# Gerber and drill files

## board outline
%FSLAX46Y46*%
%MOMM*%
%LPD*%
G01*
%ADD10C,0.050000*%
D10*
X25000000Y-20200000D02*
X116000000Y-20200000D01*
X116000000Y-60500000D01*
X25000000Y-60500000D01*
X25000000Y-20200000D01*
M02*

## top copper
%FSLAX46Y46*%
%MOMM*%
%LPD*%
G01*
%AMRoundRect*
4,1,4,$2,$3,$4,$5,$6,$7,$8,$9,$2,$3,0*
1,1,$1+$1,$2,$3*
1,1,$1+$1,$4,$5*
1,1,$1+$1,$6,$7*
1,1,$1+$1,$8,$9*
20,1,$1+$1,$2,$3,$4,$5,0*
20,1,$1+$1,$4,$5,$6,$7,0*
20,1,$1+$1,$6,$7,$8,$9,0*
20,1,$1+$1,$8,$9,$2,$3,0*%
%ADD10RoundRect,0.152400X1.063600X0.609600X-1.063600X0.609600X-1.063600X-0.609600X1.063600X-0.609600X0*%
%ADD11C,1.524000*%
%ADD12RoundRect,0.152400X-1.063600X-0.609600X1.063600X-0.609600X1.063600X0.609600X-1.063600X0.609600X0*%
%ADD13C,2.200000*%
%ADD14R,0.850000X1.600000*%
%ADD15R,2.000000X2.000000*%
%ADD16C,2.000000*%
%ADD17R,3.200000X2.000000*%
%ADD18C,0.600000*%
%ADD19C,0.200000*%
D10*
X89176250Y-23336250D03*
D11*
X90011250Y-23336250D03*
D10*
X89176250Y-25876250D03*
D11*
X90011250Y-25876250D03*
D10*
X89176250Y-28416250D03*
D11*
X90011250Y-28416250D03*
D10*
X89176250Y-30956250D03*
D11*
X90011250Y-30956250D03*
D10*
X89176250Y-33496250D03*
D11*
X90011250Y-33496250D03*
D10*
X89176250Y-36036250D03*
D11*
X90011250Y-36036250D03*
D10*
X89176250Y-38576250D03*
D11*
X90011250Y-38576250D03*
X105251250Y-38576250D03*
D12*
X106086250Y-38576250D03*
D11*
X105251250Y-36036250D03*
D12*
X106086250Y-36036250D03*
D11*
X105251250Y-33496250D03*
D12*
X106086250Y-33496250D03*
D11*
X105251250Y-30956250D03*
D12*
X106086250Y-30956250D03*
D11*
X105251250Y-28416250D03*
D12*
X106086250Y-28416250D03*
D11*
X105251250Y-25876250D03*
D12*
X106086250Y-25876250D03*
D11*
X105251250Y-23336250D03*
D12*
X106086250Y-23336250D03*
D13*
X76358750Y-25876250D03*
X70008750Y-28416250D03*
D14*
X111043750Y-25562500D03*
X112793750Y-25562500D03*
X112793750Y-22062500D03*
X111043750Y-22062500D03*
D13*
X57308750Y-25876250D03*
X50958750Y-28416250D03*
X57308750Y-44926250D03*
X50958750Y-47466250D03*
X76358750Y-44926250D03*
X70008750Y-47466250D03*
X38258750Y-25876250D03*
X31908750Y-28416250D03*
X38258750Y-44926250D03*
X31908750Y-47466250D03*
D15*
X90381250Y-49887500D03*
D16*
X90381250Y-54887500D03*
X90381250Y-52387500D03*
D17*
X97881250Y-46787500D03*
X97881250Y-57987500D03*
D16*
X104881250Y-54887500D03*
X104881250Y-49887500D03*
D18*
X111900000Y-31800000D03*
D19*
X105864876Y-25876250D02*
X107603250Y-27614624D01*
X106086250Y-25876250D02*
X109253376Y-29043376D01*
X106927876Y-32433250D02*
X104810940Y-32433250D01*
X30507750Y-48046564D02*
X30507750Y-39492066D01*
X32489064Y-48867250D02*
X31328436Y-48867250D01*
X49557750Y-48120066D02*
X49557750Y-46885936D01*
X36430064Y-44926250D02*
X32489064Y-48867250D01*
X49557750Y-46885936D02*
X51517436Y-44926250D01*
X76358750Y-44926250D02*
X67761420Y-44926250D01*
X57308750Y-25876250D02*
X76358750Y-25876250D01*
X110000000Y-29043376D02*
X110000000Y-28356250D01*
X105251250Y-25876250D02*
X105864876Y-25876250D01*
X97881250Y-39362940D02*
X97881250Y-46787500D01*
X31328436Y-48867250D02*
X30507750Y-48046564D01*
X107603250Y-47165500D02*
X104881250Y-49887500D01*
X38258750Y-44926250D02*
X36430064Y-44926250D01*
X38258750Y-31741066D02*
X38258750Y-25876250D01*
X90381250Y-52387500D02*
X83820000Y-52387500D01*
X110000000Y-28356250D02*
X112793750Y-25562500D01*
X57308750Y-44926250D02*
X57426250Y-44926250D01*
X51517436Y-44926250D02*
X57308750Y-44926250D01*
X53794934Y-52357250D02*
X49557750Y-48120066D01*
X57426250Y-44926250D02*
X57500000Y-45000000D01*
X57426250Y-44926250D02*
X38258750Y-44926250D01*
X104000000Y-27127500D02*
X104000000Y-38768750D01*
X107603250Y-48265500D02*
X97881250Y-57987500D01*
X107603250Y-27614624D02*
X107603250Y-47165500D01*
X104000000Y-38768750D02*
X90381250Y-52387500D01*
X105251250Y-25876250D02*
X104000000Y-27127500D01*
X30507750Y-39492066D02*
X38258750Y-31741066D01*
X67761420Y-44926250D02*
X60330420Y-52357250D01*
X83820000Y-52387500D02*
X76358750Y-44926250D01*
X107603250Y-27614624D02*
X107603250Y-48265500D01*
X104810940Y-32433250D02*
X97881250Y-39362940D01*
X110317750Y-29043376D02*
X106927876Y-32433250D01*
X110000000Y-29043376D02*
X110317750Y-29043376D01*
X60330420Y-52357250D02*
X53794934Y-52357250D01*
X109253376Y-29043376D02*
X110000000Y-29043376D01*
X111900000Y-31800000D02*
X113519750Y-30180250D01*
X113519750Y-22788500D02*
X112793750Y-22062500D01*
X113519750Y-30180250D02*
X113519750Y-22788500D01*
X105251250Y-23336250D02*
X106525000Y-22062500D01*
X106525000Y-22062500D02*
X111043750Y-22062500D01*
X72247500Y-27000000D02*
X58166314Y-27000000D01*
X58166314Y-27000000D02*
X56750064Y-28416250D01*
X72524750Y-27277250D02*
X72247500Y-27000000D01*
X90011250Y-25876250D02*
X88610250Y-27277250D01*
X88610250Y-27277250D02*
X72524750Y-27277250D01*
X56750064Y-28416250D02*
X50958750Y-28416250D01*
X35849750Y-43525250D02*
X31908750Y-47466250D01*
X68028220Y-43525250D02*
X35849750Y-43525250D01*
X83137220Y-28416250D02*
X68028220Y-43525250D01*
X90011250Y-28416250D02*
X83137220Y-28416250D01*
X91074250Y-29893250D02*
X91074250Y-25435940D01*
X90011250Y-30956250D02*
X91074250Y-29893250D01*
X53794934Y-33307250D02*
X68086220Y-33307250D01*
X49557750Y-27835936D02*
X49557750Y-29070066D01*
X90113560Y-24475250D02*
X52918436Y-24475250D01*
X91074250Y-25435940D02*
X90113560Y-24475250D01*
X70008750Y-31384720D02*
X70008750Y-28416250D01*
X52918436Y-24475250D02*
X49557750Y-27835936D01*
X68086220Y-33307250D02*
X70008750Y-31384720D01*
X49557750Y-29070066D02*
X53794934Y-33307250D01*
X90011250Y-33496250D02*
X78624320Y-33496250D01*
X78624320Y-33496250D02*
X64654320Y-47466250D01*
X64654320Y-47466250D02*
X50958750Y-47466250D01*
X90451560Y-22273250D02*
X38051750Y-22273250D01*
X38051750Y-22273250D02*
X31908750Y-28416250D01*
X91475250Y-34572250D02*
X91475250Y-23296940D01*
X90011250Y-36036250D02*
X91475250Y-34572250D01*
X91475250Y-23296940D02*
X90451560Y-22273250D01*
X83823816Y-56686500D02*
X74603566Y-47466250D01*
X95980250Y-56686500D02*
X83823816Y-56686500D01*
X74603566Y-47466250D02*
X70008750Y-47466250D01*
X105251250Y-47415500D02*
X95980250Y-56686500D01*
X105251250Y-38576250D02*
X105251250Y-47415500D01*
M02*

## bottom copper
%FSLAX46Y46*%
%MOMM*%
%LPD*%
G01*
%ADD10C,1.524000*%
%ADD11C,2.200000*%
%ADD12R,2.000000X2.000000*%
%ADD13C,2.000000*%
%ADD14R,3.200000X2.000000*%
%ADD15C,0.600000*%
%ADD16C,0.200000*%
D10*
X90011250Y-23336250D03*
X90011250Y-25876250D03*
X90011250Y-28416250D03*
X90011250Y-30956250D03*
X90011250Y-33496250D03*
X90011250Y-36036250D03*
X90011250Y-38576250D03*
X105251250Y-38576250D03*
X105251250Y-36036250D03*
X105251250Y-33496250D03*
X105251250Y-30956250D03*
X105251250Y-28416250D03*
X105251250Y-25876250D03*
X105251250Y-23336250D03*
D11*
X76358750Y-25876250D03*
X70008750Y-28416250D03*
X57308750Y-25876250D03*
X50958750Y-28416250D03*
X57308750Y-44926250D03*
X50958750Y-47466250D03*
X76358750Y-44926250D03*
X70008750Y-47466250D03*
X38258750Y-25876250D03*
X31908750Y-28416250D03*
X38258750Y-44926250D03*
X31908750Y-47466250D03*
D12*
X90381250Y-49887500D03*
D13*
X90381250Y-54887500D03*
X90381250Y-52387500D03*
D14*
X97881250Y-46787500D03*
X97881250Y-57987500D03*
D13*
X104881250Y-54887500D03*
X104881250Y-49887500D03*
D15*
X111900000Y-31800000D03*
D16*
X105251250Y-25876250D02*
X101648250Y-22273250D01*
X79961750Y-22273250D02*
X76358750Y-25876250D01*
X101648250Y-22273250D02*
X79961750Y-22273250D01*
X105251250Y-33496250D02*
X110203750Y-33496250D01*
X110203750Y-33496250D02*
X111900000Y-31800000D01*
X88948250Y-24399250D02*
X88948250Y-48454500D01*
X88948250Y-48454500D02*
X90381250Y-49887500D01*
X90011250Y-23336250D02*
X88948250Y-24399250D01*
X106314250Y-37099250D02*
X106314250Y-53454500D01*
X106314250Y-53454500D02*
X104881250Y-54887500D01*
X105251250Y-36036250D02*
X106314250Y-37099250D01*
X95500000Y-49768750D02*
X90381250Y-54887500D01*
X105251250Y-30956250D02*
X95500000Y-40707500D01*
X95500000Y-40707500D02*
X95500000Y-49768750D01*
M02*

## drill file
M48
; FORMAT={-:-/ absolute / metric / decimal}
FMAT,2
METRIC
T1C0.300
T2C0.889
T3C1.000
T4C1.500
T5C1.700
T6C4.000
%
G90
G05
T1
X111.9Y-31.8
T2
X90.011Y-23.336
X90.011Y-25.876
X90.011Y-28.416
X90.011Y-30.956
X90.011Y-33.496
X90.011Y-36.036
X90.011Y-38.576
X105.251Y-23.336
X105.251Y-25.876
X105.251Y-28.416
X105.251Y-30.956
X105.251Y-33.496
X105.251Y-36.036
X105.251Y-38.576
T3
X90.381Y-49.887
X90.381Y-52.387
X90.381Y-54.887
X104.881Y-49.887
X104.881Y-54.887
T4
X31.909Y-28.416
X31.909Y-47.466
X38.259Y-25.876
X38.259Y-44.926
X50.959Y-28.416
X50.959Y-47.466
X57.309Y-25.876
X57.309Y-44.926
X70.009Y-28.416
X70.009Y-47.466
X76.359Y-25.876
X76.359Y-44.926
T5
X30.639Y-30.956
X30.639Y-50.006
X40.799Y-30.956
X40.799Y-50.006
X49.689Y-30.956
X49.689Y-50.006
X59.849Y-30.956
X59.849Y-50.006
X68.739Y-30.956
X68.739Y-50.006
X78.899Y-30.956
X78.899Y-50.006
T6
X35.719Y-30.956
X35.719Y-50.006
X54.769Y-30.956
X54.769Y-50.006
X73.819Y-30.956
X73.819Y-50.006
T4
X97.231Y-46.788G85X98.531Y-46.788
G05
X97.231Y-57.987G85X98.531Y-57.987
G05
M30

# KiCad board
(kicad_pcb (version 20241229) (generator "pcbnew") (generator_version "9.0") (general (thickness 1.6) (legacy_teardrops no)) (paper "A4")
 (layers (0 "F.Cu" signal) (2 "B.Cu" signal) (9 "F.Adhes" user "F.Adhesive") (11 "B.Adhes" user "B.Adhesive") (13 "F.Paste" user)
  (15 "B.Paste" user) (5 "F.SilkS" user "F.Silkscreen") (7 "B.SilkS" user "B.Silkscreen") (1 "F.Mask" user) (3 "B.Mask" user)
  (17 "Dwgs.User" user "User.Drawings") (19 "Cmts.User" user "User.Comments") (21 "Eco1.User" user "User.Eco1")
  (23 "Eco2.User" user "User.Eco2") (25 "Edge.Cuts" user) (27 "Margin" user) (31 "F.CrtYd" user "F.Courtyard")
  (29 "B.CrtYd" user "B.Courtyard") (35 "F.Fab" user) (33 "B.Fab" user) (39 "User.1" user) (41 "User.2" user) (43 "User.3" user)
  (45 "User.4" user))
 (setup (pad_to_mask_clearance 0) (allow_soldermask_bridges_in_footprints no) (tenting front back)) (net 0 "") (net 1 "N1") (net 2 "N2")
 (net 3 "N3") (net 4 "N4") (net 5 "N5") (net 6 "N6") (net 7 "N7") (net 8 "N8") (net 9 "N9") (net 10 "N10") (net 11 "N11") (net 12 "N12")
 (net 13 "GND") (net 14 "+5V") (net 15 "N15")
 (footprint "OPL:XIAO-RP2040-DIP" (layer "F.Cu") (at 97.63125 30.95625)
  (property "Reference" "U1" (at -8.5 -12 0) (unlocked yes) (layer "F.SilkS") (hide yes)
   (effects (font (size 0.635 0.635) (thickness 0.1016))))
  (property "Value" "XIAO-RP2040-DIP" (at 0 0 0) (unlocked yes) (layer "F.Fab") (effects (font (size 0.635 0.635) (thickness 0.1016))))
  (pad "1" smd roundrect (at -8.455 -7.62 180) (size 2.432 1.524) (layers "F.Cu" "F.Mask") (roundrect_rratio 0.1) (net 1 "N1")
   (thermal_bridge_angle 45))
  (pad "1" thru_hole circle (at -7.62 -7.62 180) (size 1.524 1.524) (drill 0.889) (layers "*.Cu" "*.Mask") (remove_unused_layers no)
   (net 1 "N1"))
  (pad "2" smd roundrect (at -8.455 -5.08 180) (size 2.432 1.524) (layers "F.Cu" "F.Mask") (roundrect_rratio 0.1) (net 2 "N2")
   (thermal_bridge_angle 45))
  (pad "2" thru_hole circle (at -7.62 -5.08 180) (size 1.524 1.524) (drill 0.889) (layers "*.Cu" "*.Mask") (remove_unused_layers no)
   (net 2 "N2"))
  (pad "3" smd roundrect (at -8.455 -2.54 180) (size 2.432 1.524) (layers "F.Cu" "F.Mask") (roundrect_rratio 0.1) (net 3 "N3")
   (thermal_bridge_angle 45))
  (pad "3" thru_hole circle (at -7.62 -2.54 180) (size 1.524 1.524) (drill 0.889) (layers "*.Cu" "*.Mask") (remove_unused_layers no)
   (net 3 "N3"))
  (pad "4" smd roundrect (at -8.455 0 180) (size 2.432 1.524) (layers "F.Cu" "F.Mask") (roundrect_rratio 0.1) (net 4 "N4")
   (thermal_bridge_angle 45))
  (pad "4" thru_hole circle (at -7.62 0 180) (size 1.524 1.524) (drill 0.889) (layers "*.Cu" "*.Mask") (remove_unused_layers no)
   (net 4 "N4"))
  (pad "5" smd roundrect (at -8.455 2.54 180) (size 2.432 1.524) (layers "F.Cu" "F.Mask") (roundrect_rratio 0.1) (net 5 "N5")
   (thermal_bridge_angle 45))
  (pad "5" thru_hole circle (at -7.62 2.54 180) (size 1.524 1.524) (drill 0.889) (layers "*.Cu" "*.Mask") (remove_unused_layers no)
   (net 5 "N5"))
  (pad "6" smd roundrect (at -8.455 5.08 180) (size 2.432 1.524) (layers "F.Cu" "F.Mask") (roundrect_rratio 0.1) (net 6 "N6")
   (thermal_bridge_angle 45))
  (pad "6" thru_hole circle (at -7.62 5.08 180) (size 1.524 1.524) (drill 0.889) (layers "*.Cu" "*.Mask") (remove_unused_layers no)
   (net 6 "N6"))
  (pad "7" smd roundrect (at -8.455 7.62 180) (size 2.432 1.524) (layers "F.Cu" "F.Mask") (roundrect_rratio 0.1) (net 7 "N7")
   (thermal_bridge_angle 45))
  (pad "7" thru_hole circle (at -7.62 7.62 180) (size 1.524 1.524) (drill 0.889) (layers "*.Cu" "*.Mask") (remove_unused_layers no)
   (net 7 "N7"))
  (pad "8" thru_hole circle (at 7.62 7.62) (size 1.524 1.524) (drill 0.889) (layers "*.Cu" "*.Mask") (remove_unused_layers no) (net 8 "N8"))
  (pad "8" smd roundrect (at 8.455 7.62) (size 2.432 1.524) (layers "F.Cu" "F.Mask") (roundrect_rratio 0.1) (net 8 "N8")
   (thermal_bridge_angle 45))
  (pad "9" thru_hole circle (at 7.62 5.08) (size 1.524 1.524) (drill 0.889) (layers "*.Cu" "*.Mask") (remove_unused_layers no) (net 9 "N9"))
  (pad "9" smd roundrect (at 8.455 5.08) (size 2.432 1.524) (layers "F.Cu" "F.Mask") (roundrect_rratio 0.1) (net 9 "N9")
   (thermal_bridge_angle 45))
  (pad "10" thru_hole circle (at 7.62 2.54) (size 1.524 1.524) (drill 0.889) (layers "*.Cu" "*.Mask") (remove_unused_layers no)
   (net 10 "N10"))
  (pad "10" smd roundrect (at 8.455 2.54) (size 2.432 1.524) (layers "F.Cu" "F.Mask") (roundrect_rratio 0.1) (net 10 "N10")
   (thermal_bridge_angle 45))
  (pad "11" thru_hole circle (at 7.62 0) (size 1.524 1.524) (drill 0.889) (layers "*.Cu" "*.Mask") (remove_unused_layers no) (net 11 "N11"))
  (pad "11" smd roundrect (at 8.455 0) (size 2.432 1.524) (layers "F.Cu" "F.Mask") (roundrect_rratio 0.1) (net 11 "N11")
   (thermal_bridge_angle 45))
  (pad "12" thru_hole circle (at 7.62 -2.54) (size 1.524 1.524) (drill 0.889) (layers "*.Cu" "*.Mask") (remove_unused_layers no)
   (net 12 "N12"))
  (pad "12" smd roundrect (at 8.455 -2.54) (size 2.432 1.524) (layers "F.Cu" "F.Mask") (roundrect_rratio 0.1) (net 12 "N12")
   (thermal_bridge_angle 45))
  (pad "13" thru_hole circle (at 7.62 -5.08) (size 1.524 1.524) (drill 0.889) (layers "*.Cu" "*.Mask") (remove_unused_layers no)
   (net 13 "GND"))
  (pad "13" smd roundrect (at 8.455 -5.08) (size 2.432 1.524) (layers "F.Cu" "F.Mask") (roundrect_rratio 0.1) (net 13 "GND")
   (thermal_bridge_angle 45))
  (pad "14" thru_hole circle (at 7.62 -7.62) (size 1.524 1.524) (drill 0.889) (layers "*.Cu" "*.Mask") (remove_unused_layers no)
   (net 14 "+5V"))
  (pad "14" smd roundrect (at 8.455 -7.62) (size 2.432 1.524) (layers "F.Cu" "F.Mask") (roundrect_rratio 0.1) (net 14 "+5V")
   (thermal_bridge_angle 45)))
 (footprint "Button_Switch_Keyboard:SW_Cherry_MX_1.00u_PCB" (layer "F.Cu") (at 76.35875 25.87625)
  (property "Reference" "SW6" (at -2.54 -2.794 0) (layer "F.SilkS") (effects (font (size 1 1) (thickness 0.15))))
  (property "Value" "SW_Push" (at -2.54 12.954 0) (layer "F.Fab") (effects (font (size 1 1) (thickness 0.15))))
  (pad "" np_thru_hole circle (at -7.62 5.08) (size 1.7 1.7) (drill 1.7) (layers "*.Cu" "*.Mask"))
  (pad "" np_thru_hole circle (at -2.54 5.08) (size 4 4) (drill 4) (layers "*.Cu" "*.Mask"))
  (pad "" np_thru_hole circle (at 2.54 5.08) (size 1.7 1.7) (drill 1.7) (layers "*.Cu" "*.Mask"))
  (pad "1" thru_hole circle (at 0 0) (size 2.2 2.2) (drill 1.5) (layers "*.Cu" "*.Mask") (remove_unused_layers no) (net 13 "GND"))
  (pad "2" thru_hole circle (at -6.35 2.54) (size 2.2 2.2) (drill 1.5) (layers "*.Cu" "*.Mask") (remove_unused_layers no) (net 4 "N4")))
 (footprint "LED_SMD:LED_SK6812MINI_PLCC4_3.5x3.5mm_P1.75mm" (layer "F.Cu") (at 111.91875 23.8125 90)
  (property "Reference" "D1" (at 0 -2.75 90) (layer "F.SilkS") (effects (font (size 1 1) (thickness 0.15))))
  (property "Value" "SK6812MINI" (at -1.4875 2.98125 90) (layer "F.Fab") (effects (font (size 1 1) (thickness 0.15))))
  (pad "1" smd rect (at -1.75 -0.875 90) (size 1.6 0.85) (layers "F.Cu" "F.Mask" "F.Paste") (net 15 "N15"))
  (pad "2" smd rect (at -1.75 0.875 90) (size 1.6 0.85) (layers "F.Cu" "F.Mask" "F.Paste") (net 13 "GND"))
  (pad "3" smd rect (at 1.75 0.875 90) (size 1.6 0.85) (layers "F.Cu" "F.Mask" "F.Paste") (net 10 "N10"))
  (pad "4" smd rect (at 1.75 -0.875 90) (size 1.6 0.85) (layers "F.Cu" "F.Mask" "F.Paste") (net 14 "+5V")))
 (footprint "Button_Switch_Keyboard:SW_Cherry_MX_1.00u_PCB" (layer "F.Cu") (at 57.30875 25.87625)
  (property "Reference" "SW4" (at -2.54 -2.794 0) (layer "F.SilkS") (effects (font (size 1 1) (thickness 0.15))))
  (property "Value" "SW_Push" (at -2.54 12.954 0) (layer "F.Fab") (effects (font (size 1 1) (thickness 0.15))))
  (pad "" np_thru_hole circle (at -7.62 5.08) (size 1.7 1.7) (drill 1.7) (layers "*.Cu" "*.Mask"))
  (pad "" np_thru_hole circle (at -2.54 5.08) (size 4 4) (drill 4) (layers "*.Cu" "*.Mask"))
  (pad "" np_thru_hole circle (at 2.54 5.08) (size 1.7 1.7) (drill 1.7) (layers "*.Cu" "*.Mask"))
  (pad "1" thru_hole circle (at 0 0) (size 2.2 2.2) (drill 1.5) (layers "*.Cu" "*.Mask") (remove_unused_layers no) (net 13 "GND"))
  (pad "2" thru_hole circle (at -6.35 2.54) (size 2.2 2.2) (drill 1.5) (layers "*.Cu" "*.Mask") (remove_unused_layers no) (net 2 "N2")))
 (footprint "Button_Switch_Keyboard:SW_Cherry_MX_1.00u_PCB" (layer "F.Cu") (at 57.30875 44.92625)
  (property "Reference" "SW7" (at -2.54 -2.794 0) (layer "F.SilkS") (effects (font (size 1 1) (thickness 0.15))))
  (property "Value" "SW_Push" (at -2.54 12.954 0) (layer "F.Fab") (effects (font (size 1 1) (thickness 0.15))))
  (pad "" np_thru_hole circle (at -7.62 5.08) (size 1.7 1.7) (drill 1.7) (layers "*.Cu" "*.Mask"))
  (pad "" np_thru_hole circle (at -2.54 5.08) (size 4 4) (drill 4) (layers "*.Cu" "*.Mask"))
  (pad "" np_thru_hole circle (at 2.54 5.08) (size 1.7 1.7) (drill 1.7) (layers "*.Cu" "*.Mask"))
  (pad "1" thru_hole circle (at 0 0) (size 2.2 2.2) (drill 1.5) (layers "*.Cu" "*.Mask") (remove_unused_layers no) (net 13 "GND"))
  (pad "2" thru_hole circle (at -6.35 2.54) (size 2.2 2.2) (drill 1.5) (layers "*.Cu" "*.Mask") (remove_unused_layers no) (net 5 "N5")))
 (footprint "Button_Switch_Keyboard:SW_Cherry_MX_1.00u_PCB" (layer "F.Cu") (at 76.35875 44.92625)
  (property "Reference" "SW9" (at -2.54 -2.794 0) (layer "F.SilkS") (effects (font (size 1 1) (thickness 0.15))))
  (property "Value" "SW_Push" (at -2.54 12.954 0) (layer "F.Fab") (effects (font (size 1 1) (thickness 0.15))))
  (pad "" np_thru_hole circle (at -7.62 5.08) (size 1.7 1.7) (drill 1.7) (layers "*.Cu" "*.Mask"))
  (pad "" np_thru_hole circle (at -2.54 5.08) (size 4 4) (drill 4) (layers "*.Cu" "*.Mask"))
  (pad "" np_thru_hole circle (at 2.54 5.08) (size 1.7 1.7) (drill 1.7) (layers "*.Cu" "*.Mask"))
  (pad "1" thru_hole circle (at 0 0) (size 2.2 2.2) (drill 1.5) (layers "*.Cu" "*.Mask") (remove_unused_layers no) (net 13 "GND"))
  (pad "2" thru_hole circle (at -6.35 2.54) (size 2.2 2.2) (drill 1.5) (layers "*.Cu" "*.Mask") (remove_unused_layers no) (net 8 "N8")))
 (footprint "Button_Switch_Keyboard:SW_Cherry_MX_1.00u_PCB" (layer "F.Cu") (at 38.25875 25.87625)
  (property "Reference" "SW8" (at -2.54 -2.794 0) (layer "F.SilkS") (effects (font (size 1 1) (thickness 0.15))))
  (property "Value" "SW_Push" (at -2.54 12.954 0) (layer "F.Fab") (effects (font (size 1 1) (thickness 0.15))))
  (pad "" np_thru_hole circle (at -7.62 5.08) (size 1.7 1.7) (drill 1.7) (layers "*.Cu" "*.Mask"))
  (pad "" np_thru_hole circle (at -2.54 5.08) (size 4 4) (drill 4) (layers "*.Cu" "*.Mask"))
  (pad "" np_thru_hole circle (at 2.54 5.08) (size 1.7 1.7) (drill 1.7) (layers "*.Cu" "*.Mask"))
  (pad "1" thru_hole circle (at 0 0) (size 2.2 2.2) (drill 1.5) (layers "*.Cu" "*.Mask") (remove_unused_layers no) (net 13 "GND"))
  (pad "2" thru_hole circle (at -6.35 2.54) (size 2.2 2.2) (drill 1.5) (layers "*.Cu" "*.Mask") (remove_unused_layers no) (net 6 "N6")))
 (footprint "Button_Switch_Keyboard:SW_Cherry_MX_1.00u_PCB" (layer "F.Cu") (at 38.25875 44.92625)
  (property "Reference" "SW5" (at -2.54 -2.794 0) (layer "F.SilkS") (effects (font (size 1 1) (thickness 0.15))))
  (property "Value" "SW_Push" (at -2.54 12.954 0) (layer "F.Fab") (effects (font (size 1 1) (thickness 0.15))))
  (pad "" np_thru_hole circle (at -7.62 5.08) (size 1.7 1.7) (drill 1.7) (layers "*.Cu" "*.Mask"))
  (pad "" np_thru_hole circle (at -2.54 5.08) (size 4 4) (drill 4) (layers "*.Cu" "*.Mask"))
  (pad "" np_thru_hole circle (at 2.54 5.08) (size 1.7 1.7) (drill 1.7) (layers "*.Cu" "*.Mask"))
  (pad "1" thru_hole circle (at 0 0) (size 2.2 2.2) (drill 1.5) (layers "*.Cu" "*.Mask") (remove_unused_layers no) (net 13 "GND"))
  (pad "2" thru_hole circle (at -6.35 2.54) (size 2.2 2.2) (drill 1.5) (layers "*.Cu" "*.Mask") (remove_unused_layers no) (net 3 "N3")))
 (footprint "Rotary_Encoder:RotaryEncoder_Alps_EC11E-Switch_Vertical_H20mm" (layer "F.Cu") (at 90.38125 49.8875)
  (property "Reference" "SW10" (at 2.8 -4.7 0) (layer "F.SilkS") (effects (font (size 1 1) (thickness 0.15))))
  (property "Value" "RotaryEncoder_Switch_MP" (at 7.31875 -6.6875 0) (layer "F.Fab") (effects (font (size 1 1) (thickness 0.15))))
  (pad "A" thru_hole rect (at 0 0) (size 2 2) (drill 1) (layers "*.Cu" "*.Mask") (remove_unused_layers no) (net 1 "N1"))
  (pad "B" thru_hole circle (at 0 5) (size 2 2) (drill 1) (layers "*.Cu" "*.Mask") (remove_unused_layers no) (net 11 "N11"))
  (pad "C" thru_hole circle (at 0 2.5) (size 2 2) (drill 1) (layers "*.Cu" "*.Mask") (remove_unused_layers no) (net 13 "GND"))
  (pad "MP" thru_hole rect (at 7.5 -3.1) (size 3.2 2) (drill oval 2.8 1.5) (layers "*.Cu" "*.Mask") (remove_unused_layers no) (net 13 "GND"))
  (pad "MP" thru_hole rect (at 7.5 8.1) (size 3.2 2) (drill oval 2.8 1.5) (layers "*.Cu" "*.Mask") (remove_unused_layers no) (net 13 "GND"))
  (pad "S1" thru_hole circle (at 14.5 5) (size 2 2) (drill 1) (layers "*.Cu" "*.Mask") (remove_unused_layers no) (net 9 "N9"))
  (pad "S2" thru_hole circle (at 14.5 0) (size 2 2) (drill 1) (layers "*.Cu" "*.Mask") (remove_unused_layers no) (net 13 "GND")))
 (gr_rect (start 25 20.2) (end 116 60.5) (stroke (width 0.05) (type default)) (fill no) (layer "Edge.Cuts"))
 (segment (start 105.864876 25.87625) (end 107.60325 27.614624) (width 0.2) (layer "F.Cu") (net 13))
 (segment (start 106.08625 25.87625) (end 109.253376 29.043376) (width 0.2) (layer "F.Cu") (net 13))
 (segment (start 106.927876 32.43325) (end 104.81094 32.43325) (width 0.2) (layer "F.Cu") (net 13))
 (segment (start 30.50775 48.046564) (end 30.50775 39.492066) (width 0.2) (layer "F.Cu") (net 13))
 (segment (start 32.489064 48.86725) (end 31.328436 48.86725) (width 0.2) (layer "F.Cu") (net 13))
 (segment (start 49.55775 48.120066) (end 49.55775 46.885936) (width 0.2) (layer "F.Cu") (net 13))
 (segment (start 36.430064 44.92625) (end 32.489064 48.86725) (width 0.2) (layer "F.Cu") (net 13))
 (segment (start 49.55775 46.885936) (end 51.517436 44.92625) (width 0.2) (layer "F.Cu") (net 13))
 (segment (start 76.35875 44.92625) (end 67.76142 44.92625) (width 0.2) (layer "F.Cu") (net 13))
 (segment (start 57.30875 25.87625) (end 76.35875 25.87625) (width 0.2) (layer "F.Cu") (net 13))
 (segment (start 110 29.043376) (end 110 28.35625) (width 0.2) (layer "F.Cu") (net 13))
 (segment (start 105.25125 25.87625) (end 105.864876 25.87625) (width 0.2) (layer "F.Cu") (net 13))
 (segment (start 97.88125 39.36294) (end 97.88125 46.7875) (width 0.2) (layer "F.Cu") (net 13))
 (segment (start 31.328436 48.86725) (end 30.50775 48.046564) (width 0.2) (layer "F.Cu") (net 13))
 (segment (start 107.60325 47.1655) (end 104.88125 49.8875) (width 0.2) (layer "F.Cu") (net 13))
 (segment (start 38.25875 44.92625) (end 36.430064 44.92625) (width 0.2) (layer "F.Cu") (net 13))
 (segment (start 38.25875 31.741066) (end 38.25875 25.87625) (width 0.2) (layer "F.Cu") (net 13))
 (segment (start 90.38125 52.3875) (end 83.82 52.3875) (width 0.2) (layer "F.Cu") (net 13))
 (segment (start 110 28.35625) (end 112.79375 25.5625) (width 0.2) (layer "F.Cu") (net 13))
 (segment (start 57.30875 44.92625) (end 57.42625 44.92625) (width 0.2) (layer "F.Cu") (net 13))
 (segment (start 51.517436 44.92625) (end 57.30875 44.92625) (width 0.2) (layer "F.Cu") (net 13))
 (segment (start 53.794934 52.35725) (end 49.55775 48.120066) (width 0.2) (layer "F.Cu") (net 13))
 (segment (start 57.42625 44.92625) (end 57.5 45) (width 0.2) (layer "F.Cu") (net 13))
 (segment (start 57.42625 44.92625) (end 38.25875 44.92625) (width 0.2) (layer "F.Cu") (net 13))
 (segment (start 104 27.1275) (end 104 38.76875) (width 0.2) (layer "F.Cu") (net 13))
 (segment (start 107.60325 48.2655) (end 97.88125 57.9875) (width 0.2) (layer "F.Cu") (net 13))
 (segment (start 107.60325 27.614624) (end 107.60325 47.1655) (width 0.2) (layer "F.Cu") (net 13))
 (segment (start 104 38.76875) (end 90.38125 52.3875) (width 0.2) (layer "F.Cu") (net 13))
 (segment (start 105.25125 25.87625) (end 104 27.1275) (width 0.2) (layer "F.Cu") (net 13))
 (segment (start 30.50775 39.492066) (end 38.25875 31.741066) (width 0.2) (layer "F.Cu") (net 13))
 (segment (start 67.76142 44.92625) (end 60.33042 52.35725) (width 0.2) (layer "F.Cu") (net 13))
 (segment (start 83.82 52.3875) (end 76.35875 44.92625) (width 0.2) (layer "F.Cu") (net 13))
 (segment (start 107.60325 27.614624) (end 107.60325 48.2655) (width 0.2) (layer "F.Cu") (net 13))
 (segment (start 104.81094 32.43325) (end 97.88125 39.36294) (width 0.2) (layer "F.Cu") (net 13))
 (segment (start 110.31775 29.043376) (end 106.927876 32.43325) (width 0.2) (layer "F.Cu") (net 13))
 (segment (start 110 29.043376) (end 110.31775 29.043376) (width 0.2) (layer "F.Cu") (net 13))
 (segment (start 60.33042 52.35725) (end 53.794934 52.35725) (width 0.2) (layer "F.Cu") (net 13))
 (segment (start 109.253376 29.043376) (end 110 29.043376) (width 0.2) (layer "F.Cu") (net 13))
 (segment (start 105.25125 25.87625) (end 101.64825 22.27325) (width 0.2) (layer "B.Cu") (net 13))
 (segment (start 79.96175 22.27325) (end 76.35875 25.87625) (width 0.2) (layer "B.Cu") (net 13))
 (segment (start 101.64825 22.27325) (end 79.96175 22.27325) (width 0.2) (layer "B.Cu") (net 13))
 (segment (start 111.9 31.8) (end 113.51975 30.18025) (width 0.2) (layer "F.Cu") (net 10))
 (segment (start 113.51975 22.7885) (end 112.79375 22.0625) (width 0.2) (layer "F.Cu") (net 10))
 (segment (start 113.51975 30.18025) (end 113.51975 22.7885) (width 0.2) (layer "F.Cu") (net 10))
 (via (at 111.9 31.8) (size 0.6) (drill 0.3) (layers "F.Cu" "B.Cu") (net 10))
 (segment (start 105.25125 33.49625) (end 110.20375 33.49625) (width 0.2) (layer "B.Cu") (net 10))
 (segment (start 110.20375 33.49625) (end 111.9 31.8) (width 0.2) (layer "B.Cu") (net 10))
 (segment (start 105.25125 23.33625) (end 106.525 22.0625) (width 0.2) (layer "F.Cu") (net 14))
 (segment (start 106.525 22.0625) (end 111.04375 22.0625) (width 0.2) (layer "F.Cu") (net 14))
 (segment (start 72.2475 27) (end 58.166314 27) (width 0.2) (layer "F.Cu") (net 2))
 (segment (start 58.166314 27) (end 56.750064 28.41625) (width 0.2) (layer "F.Cu") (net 2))
 (segment (start 72.52475 27.27725) (end 72.2475 27) (width 0.2) (layer "F.Cu") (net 2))
 (segment (start 90.01125 25.87625) (end 88.61025 27.27725) (width 0.2) (layer "F.Cu") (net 2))
 (segment (start 88.61025 27.27725) (end 72.52475 27.27725) (width 0.2) (layer "F.Cu") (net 2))
 (segment (start 56.750064 28.41625) (end 50.95875 28.41625) (width 0.2) (layer "F.Cu") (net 2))
 (segment (start 35.84975 43.52525) (end 31.90875 47.46625) (width 0.2) (layer "F.Cu") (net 3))
 (segment (start 68.02822 43.52525) (end 35.84975 43.52525) (width 0.2) (layer "F.Cu") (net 3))
 (segment (start 83.13722 28.41625) (end 68.02822 43.52525) (width 0.2) (layer "F.Cu") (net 3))
 (segment (start 90.01125 28.41625) (end 83.13722 28.41625) (width 0.2) (layer "F.Cu") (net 3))
 (segment (start 91.07425 29.89325) (end 91.07425 25.43594) (width 0.2) (layer "F.Cu") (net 4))
 (segment (start 90.01125 30.95625) (end 91.07425 29.89325) (width 0.2) (layer "F.Cu") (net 4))
 (segment (start 53.794934 33.30725) (end 68.08622 33.30725) (width 0.2) (layer "F.Cu") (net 4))
 (segment (start 49.55775 27.835936) (end 49.55775 29.070066) (width 0.2) (layer "F.Cu") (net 4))
 (segment (start 90.11356 24.47525) (end 52.918436 24.47525) (width 0.2) (layer "F.Cu") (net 4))
 (segment (start 91.07425 25.43594) (end 90.11356 24.47525) (width 0.2) (layer "F.Cu") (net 4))
 (segment (start 70.00875 31.38472) (end 70.00875 28.41625) (width 0.2) (layer "F.Cu") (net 4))
 (segment (start 52.918436 24.47525) (end 49.55775 27.835936) (width 0.2) (layer "F.Cu") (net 4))
 (segment (start 68.08622 33.30725) (end 70.00875 31.38472) (width 0.2) (layer "F.Cu") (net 4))
 (segment (start 49.55775 29.070066) (end 53.794934 33.30725) (width 0.2) (layer "F.Cu") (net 4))
 (segment (start 90.01125 33.49625) (end 78.62432 33.49625) (width 0.2) (layer "F.Cu") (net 5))
 (segment (start 78.62432 33.49625) (end 64.65432 47.46625) (width 0.2) (layer "F.Cu") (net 5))
 (segment (start 64.65432 47.46625) (end 50.95875 47.46625) (width 0.2) (layer "F.Cu") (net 5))
 (segment (start 90.45156 22.27325) (end 38.05175 22.27325) (width 0.2) (layer "F.Cu") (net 6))
 (segment (start 38.05175 22.27325) (end 31.90875 28.41625) (width 0.2) (layer "F.Cu") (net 6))
 (segment (start 91.47525 34.57225) (end 91.47525 23.29694) (width 0.2) (layer "F.Cu") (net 6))
 (segment (start 90.01125 36.03625) (end 91.47525 34.57225) (width 0.2) (layer "F.Cu") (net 6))
 (segment (start 91.47525 23.29694) (end 90.45156 22.27325) (width 0.2) (layer "F.Cu") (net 6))
 (segment (start 83.823816 56.6865) (end 74.603566 47.46625) (width 0.2) (layer "F.Cu") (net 8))
 (segment (start 95.98025 56.6865) (end 83.823816 56.6865) (width 0.2) (layer "F.Cu") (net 8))
 (segment (start 74.603566 47.46625) (end 70.00875 47.46625) (width 0.2) (layer "F.Cu") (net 8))
 (segment (start 105.25125 47.4155) (end 95.98025 56.6865) (width 0.2) (layer "F.Cu") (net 8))
 (segment (start 105.25125 38.57625) (end 105.25125 47.4155) (width 0.2) (layer "F.Cu") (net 8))
 (segment (start 88.94825 24.39925) (end 88.94825 48.4545) (width 0.2) (layer "B.Cu") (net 1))
 (segment (start 88.94825 48.4545) (end 90.38125 49.8875) (width 0.2) (layer "B.Cu") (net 1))
 (segment (start 90.01125 23.33625) (end 88.94825 24.39925) (width 0.2) (layer "B.Cu") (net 1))
 (segment (start 106.31425 37.09925) (end 106.31425 53.4545) (width 0.2) (layer "B.Cu") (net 9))
 (segment (start 106.31425 53.4545) (end 104.88125 54.8875) (width 0.2) (layer "B.Cu") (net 9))
 (segment (start 105.25125 36.03625) (end 106.31425 37.09925) (width 0.2) (layer "B.Cu") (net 9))
 (segment (start 95.5 49.76875) (end 90.38125 54.8875) (width 0.2) (layer "B.Cu") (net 11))
 (segment (start 105.25125 30.95625) (end 95.5 40.7075) (width 0.2) (layer "B.Cu") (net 11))
 (segment (start 95.5 40.7075) (end 95.5 49.76875) (width 0.2) (layer "B.Cu") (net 11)))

